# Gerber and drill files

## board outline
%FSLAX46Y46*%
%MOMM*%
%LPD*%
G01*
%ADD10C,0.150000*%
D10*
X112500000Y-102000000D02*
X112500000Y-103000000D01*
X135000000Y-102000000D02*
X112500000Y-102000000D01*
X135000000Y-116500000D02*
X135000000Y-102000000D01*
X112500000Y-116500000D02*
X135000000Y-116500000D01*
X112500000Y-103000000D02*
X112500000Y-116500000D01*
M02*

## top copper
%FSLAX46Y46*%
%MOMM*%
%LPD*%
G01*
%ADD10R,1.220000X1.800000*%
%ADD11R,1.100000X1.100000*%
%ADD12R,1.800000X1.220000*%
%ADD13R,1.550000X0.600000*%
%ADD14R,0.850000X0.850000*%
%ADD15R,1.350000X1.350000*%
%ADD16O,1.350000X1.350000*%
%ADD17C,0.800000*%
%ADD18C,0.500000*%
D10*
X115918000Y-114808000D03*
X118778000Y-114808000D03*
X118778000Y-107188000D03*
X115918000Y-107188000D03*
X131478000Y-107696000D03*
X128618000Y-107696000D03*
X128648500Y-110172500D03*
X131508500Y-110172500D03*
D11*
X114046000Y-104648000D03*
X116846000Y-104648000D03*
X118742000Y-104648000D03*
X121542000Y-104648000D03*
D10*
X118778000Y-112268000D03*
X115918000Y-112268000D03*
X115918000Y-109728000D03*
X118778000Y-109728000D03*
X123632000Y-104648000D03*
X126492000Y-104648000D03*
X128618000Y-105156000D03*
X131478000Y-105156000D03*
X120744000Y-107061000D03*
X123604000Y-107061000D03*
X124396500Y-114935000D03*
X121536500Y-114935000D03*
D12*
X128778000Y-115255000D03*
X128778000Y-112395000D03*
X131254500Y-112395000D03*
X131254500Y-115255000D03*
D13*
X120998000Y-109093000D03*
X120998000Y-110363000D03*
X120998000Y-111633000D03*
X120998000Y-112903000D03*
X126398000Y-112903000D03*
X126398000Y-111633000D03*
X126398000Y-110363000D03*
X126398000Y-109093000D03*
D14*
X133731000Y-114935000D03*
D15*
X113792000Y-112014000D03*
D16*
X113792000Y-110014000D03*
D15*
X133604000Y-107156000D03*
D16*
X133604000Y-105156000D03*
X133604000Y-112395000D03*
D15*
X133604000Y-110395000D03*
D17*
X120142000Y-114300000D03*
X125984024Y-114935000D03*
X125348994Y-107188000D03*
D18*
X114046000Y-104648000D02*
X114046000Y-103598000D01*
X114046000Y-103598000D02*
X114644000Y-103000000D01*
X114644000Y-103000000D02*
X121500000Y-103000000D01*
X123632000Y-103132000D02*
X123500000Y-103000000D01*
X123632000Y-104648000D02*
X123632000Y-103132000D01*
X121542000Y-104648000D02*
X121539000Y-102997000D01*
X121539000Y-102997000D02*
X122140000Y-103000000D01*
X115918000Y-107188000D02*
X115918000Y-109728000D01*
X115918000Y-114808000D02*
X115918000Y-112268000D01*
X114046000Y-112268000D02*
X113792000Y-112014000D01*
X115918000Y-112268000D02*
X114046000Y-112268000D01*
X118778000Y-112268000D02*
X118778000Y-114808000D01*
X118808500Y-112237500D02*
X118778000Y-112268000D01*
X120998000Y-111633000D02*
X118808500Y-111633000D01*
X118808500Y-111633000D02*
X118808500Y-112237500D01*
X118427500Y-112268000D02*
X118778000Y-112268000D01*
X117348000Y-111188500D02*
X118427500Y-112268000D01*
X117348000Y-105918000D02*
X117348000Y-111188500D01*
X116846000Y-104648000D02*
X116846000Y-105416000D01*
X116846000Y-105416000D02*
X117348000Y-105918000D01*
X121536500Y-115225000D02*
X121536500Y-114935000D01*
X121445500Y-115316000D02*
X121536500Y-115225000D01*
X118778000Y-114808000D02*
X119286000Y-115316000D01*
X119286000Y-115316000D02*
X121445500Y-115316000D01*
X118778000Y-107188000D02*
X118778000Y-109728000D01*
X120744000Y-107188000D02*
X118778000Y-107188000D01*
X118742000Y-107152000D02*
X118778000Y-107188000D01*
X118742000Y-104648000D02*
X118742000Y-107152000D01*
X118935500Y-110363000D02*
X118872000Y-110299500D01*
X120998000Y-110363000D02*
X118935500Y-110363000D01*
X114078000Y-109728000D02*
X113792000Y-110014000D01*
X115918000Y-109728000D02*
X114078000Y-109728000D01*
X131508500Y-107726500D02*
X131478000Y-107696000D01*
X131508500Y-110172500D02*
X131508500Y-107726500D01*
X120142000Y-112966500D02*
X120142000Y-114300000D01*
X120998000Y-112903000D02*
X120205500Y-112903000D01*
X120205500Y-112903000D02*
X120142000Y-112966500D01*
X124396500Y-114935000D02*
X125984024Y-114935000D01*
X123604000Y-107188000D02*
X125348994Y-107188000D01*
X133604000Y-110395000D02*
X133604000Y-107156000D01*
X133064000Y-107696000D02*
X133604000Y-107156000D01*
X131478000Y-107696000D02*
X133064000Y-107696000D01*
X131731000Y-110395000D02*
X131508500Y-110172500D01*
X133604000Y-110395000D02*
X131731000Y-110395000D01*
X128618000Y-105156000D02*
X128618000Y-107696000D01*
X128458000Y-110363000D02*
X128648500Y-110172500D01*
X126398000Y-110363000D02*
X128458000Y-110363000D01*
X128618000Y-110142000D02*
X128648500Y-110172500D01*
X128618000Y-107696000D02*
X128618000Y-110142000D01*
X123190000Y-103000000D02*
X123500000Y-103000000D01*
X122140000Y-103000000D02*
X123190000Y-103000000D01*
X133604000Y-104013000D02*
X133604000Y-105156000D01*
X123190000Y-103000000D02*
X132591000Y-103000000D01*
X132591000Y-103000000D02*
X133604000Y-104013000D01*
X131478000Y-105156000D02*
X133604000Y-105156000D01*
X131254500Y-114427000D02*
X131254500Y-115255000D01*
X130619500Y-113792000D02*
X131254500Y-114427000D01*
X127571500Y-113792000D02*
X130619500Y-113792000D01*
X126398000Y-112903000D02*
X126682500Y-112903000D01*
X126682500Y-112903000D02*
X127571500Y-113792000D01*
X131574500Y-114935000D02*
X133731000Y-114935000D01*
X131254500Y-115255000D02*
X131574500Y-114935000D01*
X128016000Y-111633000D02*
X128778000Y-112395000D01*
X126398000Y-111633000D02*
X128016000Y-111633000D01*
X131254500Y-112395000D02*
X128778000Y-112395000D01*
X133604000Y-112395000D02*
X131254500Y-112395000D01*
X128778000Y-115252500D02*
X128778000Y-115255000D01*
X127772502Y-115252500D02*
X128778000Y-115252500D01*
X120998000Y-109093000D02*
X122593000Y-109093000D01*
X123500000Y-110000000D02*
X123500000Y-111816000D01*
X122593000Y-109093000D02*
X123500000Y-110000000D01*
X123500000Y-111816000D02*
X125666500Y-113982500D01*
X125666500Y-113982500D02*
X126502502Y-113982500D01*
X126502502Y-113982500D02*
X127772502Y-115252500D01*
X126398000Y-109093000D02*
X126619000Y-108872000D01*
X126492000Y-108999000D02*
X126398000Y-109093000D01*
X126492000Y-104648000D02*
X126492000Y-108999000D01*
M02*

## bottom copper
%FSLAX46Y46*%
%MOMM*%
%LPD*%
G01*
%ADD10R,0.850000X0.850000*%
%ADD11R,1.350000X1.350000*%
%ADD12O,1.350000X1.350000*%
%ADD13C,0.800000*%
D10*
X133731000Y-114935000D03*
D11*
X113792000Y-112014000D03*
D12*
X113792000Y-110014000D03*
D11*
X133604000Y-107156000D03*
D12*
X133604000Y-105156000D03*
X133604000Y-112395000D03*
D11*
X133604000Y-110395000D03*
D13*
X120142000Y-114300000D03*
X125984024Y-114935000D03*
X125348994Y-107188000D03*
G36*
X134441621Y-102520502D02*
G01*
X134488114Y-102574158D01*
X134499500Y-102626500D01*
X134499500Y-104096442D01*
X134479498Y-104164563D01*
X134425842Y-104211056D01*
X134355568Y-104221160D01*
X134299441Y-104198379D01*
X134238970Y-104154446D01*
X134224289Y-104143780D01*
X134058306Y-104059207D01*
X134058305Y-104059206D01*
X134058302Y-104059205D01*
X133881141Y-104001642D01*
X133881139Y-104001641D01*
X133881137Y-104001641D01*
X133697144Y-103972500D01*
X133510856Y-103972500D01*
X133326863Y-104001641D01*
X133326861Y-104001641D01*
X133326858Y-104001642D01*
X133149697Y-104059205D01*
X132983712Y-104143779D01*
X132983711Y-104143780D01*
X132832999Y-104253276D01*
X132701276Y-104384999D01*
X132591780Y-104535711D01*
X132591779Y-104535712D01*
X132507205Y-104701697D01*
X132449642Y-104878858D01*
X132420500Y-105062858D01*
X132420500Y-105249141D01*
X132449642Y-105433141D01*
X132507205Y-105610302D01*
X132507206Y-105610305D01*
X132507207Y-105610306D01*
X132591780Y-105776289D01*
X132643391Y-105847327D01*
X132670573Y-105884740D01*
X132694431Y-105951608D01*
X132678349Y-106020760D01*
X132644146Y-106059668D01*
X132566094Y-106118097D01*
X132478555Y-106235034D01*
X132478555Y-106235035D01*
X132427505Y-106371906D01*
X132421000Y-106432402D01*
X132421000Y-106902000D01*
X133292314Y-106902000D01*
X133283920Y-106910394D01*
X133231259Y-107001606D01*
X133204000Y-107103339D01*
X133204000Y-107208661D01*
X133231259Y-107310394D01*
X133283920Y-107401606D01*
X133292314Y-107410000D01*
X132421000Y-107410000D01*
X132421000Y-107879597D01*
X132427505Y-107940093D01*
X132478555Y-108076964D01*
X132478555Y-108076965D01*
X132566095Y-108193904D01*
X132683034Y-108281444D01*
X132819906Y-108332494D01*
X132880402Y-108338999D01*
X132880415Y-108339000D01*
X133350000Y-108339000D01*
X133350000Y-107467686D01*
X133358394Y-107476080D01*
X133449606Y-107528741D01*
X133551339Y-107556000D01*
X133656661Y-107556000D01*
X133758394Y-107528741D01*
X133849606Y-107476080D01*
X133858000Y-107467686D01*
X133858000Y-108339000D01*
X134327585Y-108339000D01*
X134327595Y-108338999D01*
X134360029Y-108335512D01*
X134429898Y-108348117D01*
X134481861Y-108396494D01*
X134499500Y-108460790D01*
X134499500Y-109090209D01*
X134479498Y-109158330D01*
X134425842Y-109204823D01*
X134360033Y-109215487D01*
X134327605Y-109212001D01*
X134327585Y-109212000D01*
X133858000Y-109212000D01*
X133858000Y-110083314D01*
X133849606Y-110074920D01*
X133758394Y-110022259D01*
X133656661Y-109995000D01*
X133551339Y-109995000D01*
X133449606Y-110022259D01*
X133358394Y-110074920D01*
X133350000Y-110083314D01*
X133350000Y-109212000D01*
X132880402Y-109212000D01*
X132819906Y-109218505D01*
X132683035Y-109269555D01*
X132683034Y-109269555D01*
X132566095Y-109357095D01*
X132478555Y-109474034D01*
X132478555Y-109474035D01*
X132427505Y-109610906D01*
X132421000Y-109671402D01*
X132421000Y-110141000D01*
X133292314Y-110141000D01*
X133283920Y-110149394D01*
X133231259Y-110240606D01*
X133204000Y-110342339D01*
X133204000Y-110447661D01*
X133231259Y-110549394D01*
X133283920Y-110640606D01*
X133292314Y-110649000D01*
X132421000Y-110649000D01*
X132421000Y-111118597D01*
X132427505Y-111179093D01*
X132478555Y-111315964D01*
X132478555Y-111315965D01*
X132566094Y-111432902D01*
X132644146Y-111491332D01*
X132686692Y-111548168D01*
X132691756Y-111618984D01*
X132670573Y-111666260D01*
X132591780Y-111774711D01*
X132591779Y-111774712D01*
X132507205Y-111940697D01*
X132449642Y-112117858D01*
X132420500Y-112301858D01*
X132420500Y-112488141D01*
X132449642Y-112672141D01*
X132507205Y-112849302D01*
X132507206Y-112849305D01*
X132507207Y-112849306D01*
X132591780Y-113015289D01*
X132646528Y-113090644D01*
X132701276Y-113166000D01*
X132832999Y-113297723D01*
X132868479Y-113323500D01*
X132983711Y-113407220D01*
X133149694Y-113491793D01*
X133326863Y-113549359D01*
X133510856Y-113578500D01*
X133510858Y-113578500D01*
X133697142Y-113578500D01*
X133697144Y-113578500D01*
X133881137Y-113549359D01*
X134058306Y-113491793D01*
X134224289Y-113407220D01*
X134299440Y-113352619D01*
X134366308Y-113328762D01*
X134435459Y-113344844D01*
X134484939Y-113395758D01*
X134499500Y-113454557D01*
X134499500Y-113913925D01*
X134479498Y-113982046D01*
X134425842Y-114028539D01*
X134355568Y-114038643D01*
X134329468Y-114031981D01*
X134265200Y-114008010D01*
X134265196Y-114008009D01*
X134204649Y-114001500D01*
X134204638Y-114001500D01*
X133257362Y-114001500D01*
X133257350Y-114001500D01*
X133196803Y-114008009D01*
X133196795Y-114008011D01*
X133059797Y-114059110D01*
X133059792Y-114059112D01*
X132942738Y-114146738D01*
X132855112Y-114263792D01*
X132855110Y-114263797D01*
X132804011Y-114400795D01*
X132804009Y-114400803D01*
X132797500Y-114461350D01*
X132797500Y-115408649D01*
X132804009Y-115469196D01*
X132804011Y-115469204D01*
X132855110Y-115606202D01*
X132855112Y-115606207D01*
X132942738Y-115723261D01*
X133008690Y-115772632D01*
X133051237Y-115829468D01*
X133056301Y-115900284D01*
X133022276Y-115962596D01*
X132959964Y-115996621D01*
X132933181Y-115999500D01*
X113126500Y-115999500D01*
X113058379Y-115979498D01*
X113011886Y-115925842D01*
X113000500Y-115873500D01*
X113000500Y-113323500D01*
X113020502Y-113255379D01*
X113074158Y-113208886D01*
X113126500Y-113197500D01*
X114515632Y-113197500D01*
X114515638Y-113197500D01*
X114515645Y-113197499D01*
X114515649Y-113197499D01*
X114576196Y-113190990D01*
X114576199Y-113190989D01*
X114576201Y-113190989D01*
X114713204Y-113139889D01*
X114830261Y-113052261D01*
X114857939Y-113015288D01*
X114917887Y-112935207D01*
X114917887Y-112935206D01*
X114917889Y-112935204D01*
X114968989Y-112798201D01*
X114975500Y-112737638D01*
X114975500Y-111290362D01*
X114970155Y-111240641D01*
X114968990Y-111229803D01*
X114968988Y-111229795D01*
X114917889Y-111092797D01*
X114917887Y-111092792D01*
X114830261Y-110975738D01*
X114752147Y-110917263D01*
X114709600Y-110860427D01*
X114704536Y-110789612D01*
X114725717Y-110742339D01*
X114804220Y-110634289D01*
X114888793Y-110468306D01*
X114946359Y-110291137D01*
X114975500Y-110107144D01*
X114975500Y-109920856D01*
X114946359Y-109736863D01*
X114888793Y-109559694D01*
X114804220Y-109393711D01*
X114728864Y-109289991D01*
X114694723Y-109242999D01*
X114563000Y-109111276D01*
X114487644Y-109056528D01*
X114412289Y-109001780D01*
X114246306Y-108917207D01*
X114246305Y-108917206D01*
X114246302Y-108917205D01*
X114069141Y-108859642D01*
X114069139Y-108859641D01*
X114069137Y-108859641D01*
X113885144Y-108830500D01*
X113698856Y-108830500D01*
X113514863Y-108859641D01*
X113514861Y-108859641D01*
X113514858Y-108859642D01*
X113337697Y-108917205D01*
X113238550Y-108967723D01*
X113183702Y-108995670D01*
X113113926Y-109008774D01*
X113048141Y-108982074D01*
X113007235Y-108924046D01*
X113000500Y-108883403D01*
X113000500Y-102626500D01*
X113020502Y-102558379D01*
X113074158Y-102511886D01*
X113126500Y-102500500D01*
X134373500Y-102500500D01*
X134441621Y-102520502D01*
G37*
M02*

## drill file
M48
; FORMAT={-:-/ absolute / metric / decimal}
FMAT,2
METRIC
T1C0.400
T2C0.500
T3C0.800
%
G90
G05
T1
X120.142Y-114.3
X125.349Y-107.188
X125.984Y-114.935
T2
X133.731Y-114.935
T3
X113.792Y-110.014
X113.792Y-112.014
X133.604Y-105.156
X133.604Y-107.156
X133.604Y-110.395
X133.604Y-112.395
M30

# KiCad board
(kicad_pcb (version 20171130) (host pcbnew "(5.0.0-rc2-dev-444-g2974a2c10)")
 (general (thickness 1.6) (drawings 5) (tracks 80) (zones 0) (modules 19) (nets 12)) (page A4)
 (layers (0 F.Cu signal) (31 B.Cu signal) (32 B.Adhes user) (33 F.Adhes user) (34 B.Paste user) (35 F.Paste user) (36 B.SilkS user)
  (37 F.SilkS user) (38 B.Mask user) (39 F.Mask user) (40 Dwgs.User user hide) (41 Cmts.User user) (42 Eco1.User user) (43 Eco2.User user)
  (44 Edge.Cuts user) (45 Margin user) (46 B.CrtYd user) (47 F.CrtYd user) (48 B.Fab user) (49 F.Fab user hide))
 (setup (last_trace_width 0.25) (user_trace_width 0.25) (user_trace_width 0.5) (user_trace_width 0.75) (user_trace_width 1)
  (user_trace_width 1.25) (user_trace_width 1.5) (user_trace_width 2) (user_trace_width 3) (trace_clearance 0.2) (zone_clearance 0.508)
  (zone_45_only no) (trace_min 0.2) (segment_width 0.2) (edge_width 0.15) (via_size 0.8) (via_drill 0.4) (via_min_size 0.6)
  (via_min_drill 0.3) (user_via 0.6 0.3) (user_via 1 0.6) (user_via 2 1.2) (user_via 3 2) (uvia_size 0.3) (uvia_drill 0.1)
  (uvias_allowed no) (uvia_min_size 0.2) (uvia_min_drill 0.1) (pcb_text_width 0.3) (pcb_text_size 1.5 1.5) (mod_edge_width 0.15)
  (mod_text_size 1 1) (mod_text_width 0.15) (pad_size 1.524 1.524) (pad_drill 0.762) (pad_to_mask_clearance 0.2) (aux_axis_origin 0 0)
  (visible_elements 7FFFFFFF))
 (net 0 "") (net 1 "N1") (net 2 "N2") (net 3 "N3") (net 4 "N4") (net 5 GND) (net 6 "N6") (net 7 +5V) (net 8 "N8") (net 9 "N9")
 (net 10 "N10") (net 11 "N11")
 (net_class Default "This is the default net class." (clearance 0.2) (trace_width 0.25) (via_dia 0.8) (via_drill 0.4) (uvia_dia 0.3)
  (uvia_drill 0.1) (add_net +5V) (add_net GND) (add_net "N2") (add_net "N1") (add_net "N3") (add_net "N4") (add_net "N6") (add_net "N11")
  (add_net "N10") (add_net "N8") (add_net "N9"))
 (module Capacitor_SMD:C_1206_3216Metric (layer F.Cu) (at 117.348 114.808 180)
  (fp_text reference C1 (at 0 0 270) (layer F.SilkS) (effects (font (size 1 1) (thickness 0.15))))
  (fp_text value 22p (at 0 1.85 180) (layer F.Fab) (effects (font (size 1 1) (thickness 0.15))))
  (pad 2 smd rect (at 1.43 0 180) (size 1.22 1.8) (layers F.Cu F.Paste F.Mask) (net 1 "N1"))
  (pad 1 smd rect (at -1.43 0 180) (size 1.22 1.8) (layers F.Cu F.Paste F.Mask) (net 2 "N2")))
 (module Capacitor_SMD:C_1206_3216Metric (layer F.Cu) (at 117.348 107.188 180)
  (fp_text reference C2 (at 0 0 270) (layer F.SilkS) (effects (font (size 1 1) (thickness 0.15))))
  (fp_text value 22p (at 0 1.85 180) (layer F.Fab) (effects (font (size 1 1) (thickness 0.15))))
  (pad 1 smd rect (at -1.43 0 180) (size 1.22 1.8) (layers F.Cu F.Paste F.Mask) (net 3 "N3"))
  (pad 2 smd rect (at 1.43 0 180) (size 1.22 1.8) (layers F.Cu F.Paste F.Mask) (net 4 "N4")))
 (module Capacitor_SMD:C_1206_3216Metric (layer F.Cu) (at 130.048 107.696)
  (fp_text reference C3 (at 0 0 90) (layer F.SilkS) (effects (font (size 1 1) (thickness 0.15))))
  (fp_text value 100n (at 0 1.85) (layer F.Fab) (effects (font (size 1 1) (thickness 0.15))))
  (pad 2 smd rect (at 1.43 0) (size 1.22 1.8) (layers F.Cu F.Paste F.Mask) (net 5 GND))
  (pad 1 smd rect (at -1.43 0) (size 1.22 1.8) (layers F.Cu F.Paste F.Mask) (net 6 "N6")))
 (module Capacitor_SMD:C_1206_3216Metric (layer F.Cu) (at 130.0785 110.1725)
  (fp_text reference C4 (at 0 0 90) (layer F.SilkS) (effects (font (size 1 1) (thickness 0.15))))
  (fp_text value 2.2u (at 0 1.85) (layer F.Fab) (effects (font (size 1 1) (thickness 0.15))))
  (pad 1 smd rect (at -1.43 0) (size 1.22 1.8) (layers F.Cu F.Paste F.Mask) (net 6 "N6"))
  (pad 2 smd rect (at 1.43 0) (size 1.22 1.8) (layers F.Cu F.Paste F.Mask) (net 5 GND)))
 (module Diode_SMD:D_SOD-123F (layer F.Cu) (at 115.446 104.648)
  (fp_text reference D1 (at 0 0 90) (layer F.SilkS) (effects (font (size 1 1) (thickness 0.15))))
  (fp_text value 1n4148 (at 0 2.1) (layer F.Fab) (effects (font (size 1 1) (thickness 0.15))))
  (pad 1 smd rect (at -1.4 0) (size 1.1 1.1) (layers F.Cu F.Paste F.Mask) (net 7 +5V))
  (pad 2 smd rect (at 1.4 0) (size 1.1 1.1) (layers F.Cu F.Paste F.Mask) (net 2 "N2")))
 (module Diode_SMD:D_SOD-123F (layer F.Cu) (at 120.142 104.648 180)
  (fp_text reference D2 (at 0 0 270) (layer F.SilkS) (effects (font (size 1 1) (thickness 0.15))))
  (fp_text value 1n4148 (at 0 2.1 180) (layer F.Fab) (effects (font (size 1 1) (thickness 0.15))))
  (pad 2 smd rect (at 1.4 0 180) (size 1.1 1.1) (layers F.Cu F.Paste F.Mask) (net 3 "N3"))
  (pad 1 smd rect (at -1.4 0 180) (size 1.1 1.1) (layers F.Cu F.Paste F.Mask) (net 7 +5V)))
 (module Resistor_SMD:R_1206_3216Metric (layer F.Cu) (at 117.348 112.268 180)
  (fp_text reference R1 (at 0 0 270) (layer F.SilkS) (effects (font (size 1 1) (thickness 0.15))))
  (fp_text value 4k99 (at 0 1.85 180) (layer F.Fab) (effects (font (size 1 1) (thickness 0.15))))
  (pad 1 smd rect (at -1.43 0 180) (size 1.22 1.8) (layers F.Cu F.Paste F.Mask) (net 2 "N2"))
  (pad 2 smd rect (at 1.43 0 180) (size 1.22 1.8) (layers F.Cu F.Paste F.Mask) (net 1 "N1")))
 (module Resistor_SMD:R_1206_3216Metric (layer F.Cu) (at 117.348 109.728 180)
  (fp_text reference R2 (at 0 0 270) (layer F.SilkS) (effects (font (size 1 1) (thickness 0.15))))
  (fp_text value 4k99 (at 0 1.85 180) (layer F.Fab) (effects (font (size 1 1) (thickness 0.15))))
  (pad 2 smd rect (at 1.43 0 180) (size 1.22 1.8) (layers F.Cu F.Paste F.Mask) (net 4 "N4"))
  (pad 1 smd rect (at -1.43 0 180) (size 1.22 1.8) (layers F.Cu F.Paste F.Mask) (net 3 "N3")))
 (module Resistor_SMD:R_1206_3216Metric (layer F.Cu) (at 125.062 104.648 180)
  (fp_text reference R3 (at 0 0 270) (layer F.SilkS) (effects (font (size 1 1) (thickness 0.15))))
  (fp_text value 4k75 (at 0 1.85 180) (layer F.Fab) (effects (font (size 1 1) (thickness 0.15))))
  (pad 2 smd rect (at 1.43 0 180) (size 1.22 1.8) (layers F.Cu F.Paste F.Mask) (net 7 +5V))
  (pad 1 smd rect (at -1.43 0 180) (size 1.22 1.8) (layers F.Cu F.Paste F.Mask) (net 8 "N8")))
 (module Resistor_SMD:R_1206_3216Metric (layer F.Cu) (at 130.048 105.156)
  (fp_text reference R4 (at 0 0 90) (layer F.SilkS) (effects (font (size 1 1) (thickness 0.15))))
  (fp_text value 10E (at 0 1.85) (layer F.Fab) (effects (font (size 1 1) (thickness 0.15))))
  (pad 1 smd rect (at -1.43 0) (size 1.22 1.8) (layers F.Cu F.Paste F.Mask) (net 6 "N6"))
  (pad 2 smd rect (at 1.43 0) (size 1.22 1.8) (layers F.Cu F.Paste F.Mask) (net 7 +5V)))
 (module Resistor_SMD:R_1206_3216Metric (layer F.Cu) (at 122.174 107.061 180)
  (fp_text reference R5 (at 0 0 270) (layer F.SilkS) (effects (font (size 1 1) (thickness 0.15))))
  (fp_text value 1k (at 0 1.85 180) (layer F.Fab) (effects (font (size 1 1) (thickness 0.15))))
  (pad 2 smd rect (at 1.43 0 180) (size 1.22 1.8) (layers F.Cu F.Paste F.Mask) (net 3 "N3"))
  (pad 1 smd rect (at -1.43 0 180) (size 1.22 1.8) (layers F.Cu F.Paste F.Mask) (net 5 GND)))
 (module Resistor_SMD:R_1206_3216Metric (layer F.Cu) (at 122.9665 114.935 180)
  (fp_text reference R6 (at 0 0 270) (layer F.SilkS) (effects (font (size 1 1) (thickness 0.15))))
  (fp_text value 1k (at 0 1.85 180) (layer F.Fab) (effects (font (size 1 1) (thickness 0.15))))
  (pad 1 smd rect (at -1.43 0 180) (size 1.22 1.8) (layers F.Cu F.Paste F.Mask) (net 5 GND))
  (pad 2 smd rect (at 1.43 0 180) (size 1.22 1.8) (layers F.Cu F.Paste F.Mask) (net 2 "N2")))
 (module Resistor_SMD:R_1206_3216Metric (layer F.Cu) (at 128.778 113.825 90)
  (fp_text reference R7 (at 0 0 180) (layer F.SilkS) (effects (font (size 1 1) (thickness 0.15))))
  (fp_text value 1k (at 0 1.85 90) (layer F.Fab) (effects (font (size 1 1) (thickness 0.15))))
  (pad 1 smd rect (at -1.43 0 90) (size 1.22 1.8) (layers F.Cu F.Paste F.Mask) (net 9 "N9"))
  (pad 2 smd rect (at 1.43 0 90) (size 1.22 1.8) (layers F.Cu F.Paste F.Mask) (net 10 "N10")))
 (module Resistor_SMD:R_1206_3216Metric (layer F.Cu) (at 131.2545 113.825 90)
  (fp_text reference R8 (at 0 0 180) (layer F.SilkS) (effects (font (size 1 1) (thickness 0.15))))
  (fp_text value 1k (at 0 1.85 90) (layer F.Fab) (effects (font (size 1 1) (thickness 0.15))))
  (pad 2 smd rect (at 1.43 0 90) (size 1.22 1.8) (layers F.Cu F.Paste F.Mask) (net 10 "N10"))
  (pad 1 smd rect (at -1.43 0 90) (size 1.22 1.8) (layers F.Cu F.Paste F.Mask) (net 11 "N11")))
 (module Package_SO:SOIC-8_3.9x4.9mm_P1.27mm (layer F.Cu) (at 123.698 110.998)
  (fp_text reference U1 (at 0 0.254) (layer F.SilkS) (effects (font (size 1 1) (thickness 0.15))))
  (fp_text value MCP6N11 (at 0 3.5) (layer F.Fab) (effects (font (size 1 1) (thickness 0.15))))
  (pad 1 smd rect (at -2.7 -1.905) (size 1.55 0.6) (layers F.Cu F.Paste F.Mask) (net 9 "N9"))
  (pad 2 smd rect (at -2.7 -0.635) (size 1.55 0.6) (layers F.Cu F.Paste F.Mask) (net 3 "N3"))
  (pad 3 smd rect (at -2.7 0.635) (size 1.55 0.6) (layers F.Cu F.Paste F.Mask) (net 2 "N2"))
  (pad 4 smd rect (at -2.7 1.905) (size 1.55 0.6) (layers F.Cu F.Paste F.Mask) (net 5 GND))
  (pad 5 smd rect (at 2.7 1.905) (size 1.55 0.6) (layers F.Cu F.Paste F.Mask) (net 11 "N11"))
  (pad 6 smd rect (at 2.7 0.635) (size 1.55 0.6) (layers F.Cu F.Paste F.Mask) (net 10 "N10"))
  (pad 7 smd rect (at 2.7 -0.635) (size 1.55 0.6) (layers F.Cu F.Paste F.Mask) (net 6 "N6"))
  (pad 8 smd rect (at 2.7 -1.905) (size 1.55 0.6) (layers F.Cu F.Paste F.Mask) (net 8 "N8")))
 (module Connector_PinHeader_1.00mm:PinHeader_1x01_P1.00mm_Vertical (layer F.Cu) (at 133.731 114.935 270)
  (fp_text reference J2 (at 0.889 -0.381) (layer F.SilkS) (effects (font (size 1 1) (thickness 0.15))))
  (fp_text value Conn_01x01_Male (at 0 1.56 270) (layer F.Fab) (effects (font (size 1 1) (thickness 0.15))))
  (pad 1 thru_hole rect (at 0 0 270) (size 0.85 0.85) (drill 0.5) (layers *.Cu *.Mask) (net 11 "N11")))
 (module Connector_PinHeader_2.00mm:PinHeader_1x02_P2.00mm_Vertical (layer F.Cu) (at 113.792 112.014 180)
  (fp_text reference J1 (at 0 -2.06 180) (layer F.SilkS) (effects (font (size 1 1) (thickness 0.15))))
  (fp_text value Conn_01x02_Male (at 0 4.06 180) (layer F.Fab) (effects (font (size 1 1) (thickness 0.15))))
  (pad 1 thru_hole rect (at 0 0 180) (size 1.35 1.35) (drill 0.8) (layers *.Cu *.Mask) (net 1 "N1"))
  (pad 2 thru_hole oval (at 0 2 180) (size 1.35 1.35) (drill 0.8) (layers *.Cu *.Mask) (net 4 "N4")))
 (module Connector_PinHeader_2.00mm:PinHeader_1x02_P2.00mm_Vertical (layer F.Cu) (at 133.604 107.156 180)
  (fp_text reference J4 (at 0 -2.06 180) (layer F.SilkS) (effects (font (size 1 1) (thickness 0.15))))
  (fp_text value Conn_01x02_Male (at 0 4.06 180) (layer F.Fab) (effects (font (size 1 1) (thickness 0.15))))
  (pad 1 thru_hole rect (at 0 0 180) (size 1.35 1.35) (drill 0.8) (layers *.Cu *.Mask) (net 5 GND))
  (pad 2 thru_hole oval (at 0 2 180) (size 1.35 1.35) (drill 0.8) (layers *.Cu *.Mask) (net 7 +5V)))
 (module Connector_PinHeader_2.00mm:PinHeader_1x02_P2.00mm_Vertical (layer F.Cu) (at 133.604 110.395)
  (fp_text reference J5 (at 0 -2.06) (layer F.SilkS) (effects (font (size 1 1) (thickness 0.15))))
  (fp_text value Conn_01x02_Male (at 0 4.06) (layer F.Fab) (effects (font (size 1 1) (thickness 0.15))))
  (pad 2 thru_hole oval (at 0 2) (size 1.35 1.35) (drill 0.8) (layers *.Cu *.Mask) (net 10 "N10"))
  (pad 1 thru_hole rect (at 0 0) (size 1.35 1.35) (drill 0.8) (layers *.Cu *.Mask) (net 5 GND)))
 (gr_line (start 112.5 102) (end 112.5 103) (layer Edge.Cuts) (width 0.15))
 (gr_line (start 135 102) (end 112.5 102) (layer Edge.Cuts) (width 0.15))
 (gr_line (start 135 116.5) (end 135 102) (layer Edge.Cuts) (width 0.15))
 (gr_line (start 112.5 116.5) (end 135 116.5) (layer Edge.Cuts) (width 0.15))
 (gr_line (start 112.5 103) (end 112.5 116.5) (layer Edge.Cuts) (width 0.15))
 (segment (start 114.046 104.648) (end 114.046 103.598) (width 0.5) (layer F.Cu) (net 7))
 (segment (start 114.046 103.598) (end 114.644 103) (width 0.5) (layer F.Cu) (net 7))
 (segment (start 114.644 103) (end 121.5 103) (width 0.5) (layer F.Cu) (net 7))
 (segment (start 123.632 103.132) (end 123.5 103) (width 0.5) (layer F.Cu) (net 7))
 (segment (start 123.632 104.648) (end 123.632 103.132) (width 0.5) (layer F.Cu) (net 7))
 (segment (start 121.542 104.648) (end 121.539 102.997) (width 0.5) (layer F.Cu) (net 7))
 (segment (start 121.539 102.997) (end 122.14 103) (width 0.5) (layer F.Cu) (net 7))
 (segment (start 115.918 107.188) (end 115.918 109.728) (width 0.5) (layer F.Cu) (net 4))
 (segment (start 115.918 114.808) (end 115.918 112.268) (width 0.5) (layer F.Cu) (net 1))
 (segment (start 114.046 112.268) (end 113.792 112.014) (width 0.5) (layer F.Cu) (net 1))
 (segment (start 115.918 112.268) (end 114.046 112.268) (width 0.5) (layer F.Cu) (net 1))
 (segment (start 118.778 112.268) (end 118.778 114.808) (width 0.5) (layer F.Cu) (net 2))
 (segment (start 118.8085 112.2375) (end 118.778 112.268) (width 0.5) (layer F.Cu) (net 2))
 (segment (start 120.998 111.633) (end 118.8085 111.633) (width 0.5) (layer F.Cu) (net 2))
 (segment (start 118.8085 111.633) (end 118.8085 112.2375) (width 0.5) (layer F.Cu) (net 2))
 (segment (start 118.4275 112.268) (end 118.778 112.268) (width 0.5) (layer F.Cu) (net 2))
 (segment (start 117.348 111.1885) (end 118.4275 112.268) (width 0.5) (layer F.Cu) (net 2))
 (segment (start 117.348 105.918) (end 117.348 111.1885) (width 0.5) (layer F.Cu) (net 2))
 (segment (start 116.846 104.648) (end 116.846 105.416) (width 0.5) (layer F.Cu) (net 2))
 (segment (start 116.846 105.416) (end 117.348 105.918) (width 0.5) (layer F.Cu) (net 2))
 (segment (start 121.5365 115.225) (end 121.5365 114.935) (width 0.5) (layer F.Cu) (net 2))
 (segment (start 121.4455 115.316) (end 121.5365 115.225) (width 0.5) (layer F.Cu) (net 2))
 (segment (start 118.778 114.808) (end 119.286 115.316) (width 0.5) (layer F.Cu) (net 2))
 (segment (start 119.286 115.316) (end 121.4455 115.316) (width 0.5) (layer F.Cu) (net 2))
 (segment (start 118.778 107.188) (end 118.778 109.728) (width 0.5) (layer F.Cu) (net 3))
 (segment (start 120.744 107.188) (end 118.778 107.188) (width 0.5) (layer F.Cu) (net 3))
 (segment (start 118.742 107.152) (end 118.778 107.188) (width 0.5) (layer F.Cu) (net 3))
 (segment (start 118.742 104.648) (end 118.742 107.152) (width 0.5) (layer F.Cu) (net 3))
 (segment (start 118.9355 110.363) (end 118.872 110.2995) (width 0.5) (layer F.Cu) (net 3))
 (segment (start 120.998 110.363) (end 118.9355 110.363) (width 0.5) (layer F.Cu) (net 3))
 (segment (start 114.078 109.728) (end 113.792 110.014) (width 0.5) (layer F.Cu) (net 4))
 (segment (start 115.918 109.728) (end 114.078 109.728) (width 0.5) (layer F.Cu) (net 4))
 (segment (start 131.5085 107.7265) (end 131.478 107.696) (width 0.5) (layer F.Cu) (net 5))
 (segment (start 131.5085 110.1725) (end 131.5085 107.7265) (width 0.5) (layer F.Cu) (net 5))
 (via (at 120.142 114.3) (size 0.8) (drill 0.4) (layers F.Cu B.Cu) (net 5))
 (segment (start 120.142 112.9665) (end 120.142 114.3) (width 0.5) (layer F.Cu) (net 5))
 (segment (start 120.998 112.903) (end 120.2055 112.903) (width 0.5) (layer F.Cu) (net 5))
 (segment (start 120.2055 112.903) (end 120.142 112.9665) (width 0.5) (layer F.Cu) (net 5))
 (via (at 125.984024 114.935) (size 0.8) (drill 0.4) (layers F.Cu B.Cu) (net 5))
 (segment (start 124.3965 114.935) (end 125.984024 114.935) (width 0.5) (layer F.Cu) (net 5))
 (via (at 125.348994 107.188) (size 0.8) (drill 0.4) (layers F.Cu B.Cu) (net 5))
 (segment (start 123.604 107.188) (end 125.348994 107.188) (width 0.5) (layer F.Cu) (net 5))
 (segment (start 133.604 110.395) (end 133.604 107.156) (width 0.5) (layer F.Cu) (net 5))
 (segment (start 133.064 107.696) (end 133.604 107.156) (width 0.5) (layer F.Cu) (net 5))
 (segment (start 131.478 107.696) (end 133.064 107.696) (width 0.5) (layer F.Cu) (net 5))
 (segment (start 131.731 110.395) (end 131.5085 110.1725) (width 0.5) (layer F.Cu) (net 5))
 (segment (start 133.604 110.395) (end 131.731 110.395) (width 0.5) (layer F.Cu) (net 5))
 (segment (start 128.618 105.156) (end 128.618 107.696) (width 0.5) (layer F.Cu) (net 6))
 (segment (start 128.458 110.363) (end 128.6485 110.1725) (width 0.5) (layer F.Cu) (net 6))
 (segment (start 126.398 110.363) (end 128.458 110.363) (width 0.5) (layer F.Cu) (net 6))
 (segment (start 128.618 110.142) (end 128.6485 110.1725) (width 0.5) (layer F.Cu) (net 6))
 (segment (start 128.618 107.696) (end 128.618 110.142) (width 0.5) (layer F.Cu) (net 6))
 (segment (start 123.19 103) (end 123.5 103) (width 0.5) (layer F.Cu) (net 7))
 (segment (start 122.14 103) (end 123.19 103) (width 0.5) (layer F.Cu) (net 7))
 (segment (start 133.604 104.013) (end 133.604 105.156) (width 0.5) (layer F.Cu) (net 7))
 (segment (start 123.19 103) (end 132.591 103) (width 0.5) (layer F.Cu) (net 7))
 (segment (start 132.591 103) (end 133.604 104.013) (width 0.5) (layer F.Cu) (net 7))
 (segment (start 131.478 105.156) (end 133.604 105.156) (width 0.5) (layer F.Cu) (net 7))
 (segment (start 131.2545 114.427) (end 131.2545 115.255) (width 0.5) (layer F.Cu) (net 11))
 (segment (start 130.6195 113.792) (end 131.2545 114.427) (width 0.5) (layer F.Cu) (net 11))
 (segment (start 127.5715 113.792) (end 130.6195 113.792) (width 0.5) (layer F.Cu) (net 11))
 (segment (start 126.398 112.903) (end 126.6825 112.903) (width 0.5) (layer F.Cu) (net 11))
 (segment (start 126.6825 112.903) (end 127.5715 113.792) (width 0.5) (layer F.Cu) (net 11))
 (segment (start 131.5745 114.935) (end 133.731 114.935) (width 0.5) (layer F.Cu) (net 11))
 (segment (start 131.2545 115.255) (end 131.5745 114.935) (width 0.5) (layer F.Cu) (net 11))
 (segment (start 128.016 111.633) (end 128.778 112.395) (width 0.5) (layer F.Cu) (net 10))
 (segment (start 126.398 111.633) (end 128.016 111.633) (width 0.5) (layer F.Cu) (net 10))
 (segment (start 131.2545 112.395) (end 128.778 112.395) (width 0.5) (layer F.Cu) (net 10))
 (segment (start 133.604 112.395) (end 131.2545 112.395) (width 0.5) (layer F.Cu) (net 10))
 (segment (start 128.778 115.2525) (end 128.778 115.255) (width 0.5) (layer F.Cu) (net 9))
 (segment (start 127.772502 115.2525) (end 128.778 115.2525) (width 0.5) (layer F.Cu) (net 9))
 (segment (start 120.998 109.093) (end 122.593 109.093) (width 0.5) (layer F.Cu) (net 9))
 (segment (start 123.5 110) (end 123.5 111.816) (width 0.5) (layer F.Cu) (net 9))
 (segment (start 122.593 109.093) (end 123.5 110) (width 0.5) (layer F.Cu) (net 9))
 (segment (start 123.5 111.816) (end 125.6665 113.9825) (width 0.5) (layer F.Cu) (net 9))
 (segment (start 125.6665 113.9825) (end 126.502502 113.9825) (width 0.5) (layer F.Cu) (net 9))
 (segment (start 126.502502 113.9825) (end 127.772502 115.2525) (width 0.5) (layer F.Cu) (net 9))
 (segment (start 126.398 109.093) (end 126.619 108.872) (width 0.5) (layer F.Cu) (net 8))
 (segment (start 126.492 108.999) (end 126.398 109.093) (width 0.5) (layer F.Cu) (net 8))
 (segment (start 126.492 104.648) (end 126.492 108.999) (width 0.5) (layer F.Cu) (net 8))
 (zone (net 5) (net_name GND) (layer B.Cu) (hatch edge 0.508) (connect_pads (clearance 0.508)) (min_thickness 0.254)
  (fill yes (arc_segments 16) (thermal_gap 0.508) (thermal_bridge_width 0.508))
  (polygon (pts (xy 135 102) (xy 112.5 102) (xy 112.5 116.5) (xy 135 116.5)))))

